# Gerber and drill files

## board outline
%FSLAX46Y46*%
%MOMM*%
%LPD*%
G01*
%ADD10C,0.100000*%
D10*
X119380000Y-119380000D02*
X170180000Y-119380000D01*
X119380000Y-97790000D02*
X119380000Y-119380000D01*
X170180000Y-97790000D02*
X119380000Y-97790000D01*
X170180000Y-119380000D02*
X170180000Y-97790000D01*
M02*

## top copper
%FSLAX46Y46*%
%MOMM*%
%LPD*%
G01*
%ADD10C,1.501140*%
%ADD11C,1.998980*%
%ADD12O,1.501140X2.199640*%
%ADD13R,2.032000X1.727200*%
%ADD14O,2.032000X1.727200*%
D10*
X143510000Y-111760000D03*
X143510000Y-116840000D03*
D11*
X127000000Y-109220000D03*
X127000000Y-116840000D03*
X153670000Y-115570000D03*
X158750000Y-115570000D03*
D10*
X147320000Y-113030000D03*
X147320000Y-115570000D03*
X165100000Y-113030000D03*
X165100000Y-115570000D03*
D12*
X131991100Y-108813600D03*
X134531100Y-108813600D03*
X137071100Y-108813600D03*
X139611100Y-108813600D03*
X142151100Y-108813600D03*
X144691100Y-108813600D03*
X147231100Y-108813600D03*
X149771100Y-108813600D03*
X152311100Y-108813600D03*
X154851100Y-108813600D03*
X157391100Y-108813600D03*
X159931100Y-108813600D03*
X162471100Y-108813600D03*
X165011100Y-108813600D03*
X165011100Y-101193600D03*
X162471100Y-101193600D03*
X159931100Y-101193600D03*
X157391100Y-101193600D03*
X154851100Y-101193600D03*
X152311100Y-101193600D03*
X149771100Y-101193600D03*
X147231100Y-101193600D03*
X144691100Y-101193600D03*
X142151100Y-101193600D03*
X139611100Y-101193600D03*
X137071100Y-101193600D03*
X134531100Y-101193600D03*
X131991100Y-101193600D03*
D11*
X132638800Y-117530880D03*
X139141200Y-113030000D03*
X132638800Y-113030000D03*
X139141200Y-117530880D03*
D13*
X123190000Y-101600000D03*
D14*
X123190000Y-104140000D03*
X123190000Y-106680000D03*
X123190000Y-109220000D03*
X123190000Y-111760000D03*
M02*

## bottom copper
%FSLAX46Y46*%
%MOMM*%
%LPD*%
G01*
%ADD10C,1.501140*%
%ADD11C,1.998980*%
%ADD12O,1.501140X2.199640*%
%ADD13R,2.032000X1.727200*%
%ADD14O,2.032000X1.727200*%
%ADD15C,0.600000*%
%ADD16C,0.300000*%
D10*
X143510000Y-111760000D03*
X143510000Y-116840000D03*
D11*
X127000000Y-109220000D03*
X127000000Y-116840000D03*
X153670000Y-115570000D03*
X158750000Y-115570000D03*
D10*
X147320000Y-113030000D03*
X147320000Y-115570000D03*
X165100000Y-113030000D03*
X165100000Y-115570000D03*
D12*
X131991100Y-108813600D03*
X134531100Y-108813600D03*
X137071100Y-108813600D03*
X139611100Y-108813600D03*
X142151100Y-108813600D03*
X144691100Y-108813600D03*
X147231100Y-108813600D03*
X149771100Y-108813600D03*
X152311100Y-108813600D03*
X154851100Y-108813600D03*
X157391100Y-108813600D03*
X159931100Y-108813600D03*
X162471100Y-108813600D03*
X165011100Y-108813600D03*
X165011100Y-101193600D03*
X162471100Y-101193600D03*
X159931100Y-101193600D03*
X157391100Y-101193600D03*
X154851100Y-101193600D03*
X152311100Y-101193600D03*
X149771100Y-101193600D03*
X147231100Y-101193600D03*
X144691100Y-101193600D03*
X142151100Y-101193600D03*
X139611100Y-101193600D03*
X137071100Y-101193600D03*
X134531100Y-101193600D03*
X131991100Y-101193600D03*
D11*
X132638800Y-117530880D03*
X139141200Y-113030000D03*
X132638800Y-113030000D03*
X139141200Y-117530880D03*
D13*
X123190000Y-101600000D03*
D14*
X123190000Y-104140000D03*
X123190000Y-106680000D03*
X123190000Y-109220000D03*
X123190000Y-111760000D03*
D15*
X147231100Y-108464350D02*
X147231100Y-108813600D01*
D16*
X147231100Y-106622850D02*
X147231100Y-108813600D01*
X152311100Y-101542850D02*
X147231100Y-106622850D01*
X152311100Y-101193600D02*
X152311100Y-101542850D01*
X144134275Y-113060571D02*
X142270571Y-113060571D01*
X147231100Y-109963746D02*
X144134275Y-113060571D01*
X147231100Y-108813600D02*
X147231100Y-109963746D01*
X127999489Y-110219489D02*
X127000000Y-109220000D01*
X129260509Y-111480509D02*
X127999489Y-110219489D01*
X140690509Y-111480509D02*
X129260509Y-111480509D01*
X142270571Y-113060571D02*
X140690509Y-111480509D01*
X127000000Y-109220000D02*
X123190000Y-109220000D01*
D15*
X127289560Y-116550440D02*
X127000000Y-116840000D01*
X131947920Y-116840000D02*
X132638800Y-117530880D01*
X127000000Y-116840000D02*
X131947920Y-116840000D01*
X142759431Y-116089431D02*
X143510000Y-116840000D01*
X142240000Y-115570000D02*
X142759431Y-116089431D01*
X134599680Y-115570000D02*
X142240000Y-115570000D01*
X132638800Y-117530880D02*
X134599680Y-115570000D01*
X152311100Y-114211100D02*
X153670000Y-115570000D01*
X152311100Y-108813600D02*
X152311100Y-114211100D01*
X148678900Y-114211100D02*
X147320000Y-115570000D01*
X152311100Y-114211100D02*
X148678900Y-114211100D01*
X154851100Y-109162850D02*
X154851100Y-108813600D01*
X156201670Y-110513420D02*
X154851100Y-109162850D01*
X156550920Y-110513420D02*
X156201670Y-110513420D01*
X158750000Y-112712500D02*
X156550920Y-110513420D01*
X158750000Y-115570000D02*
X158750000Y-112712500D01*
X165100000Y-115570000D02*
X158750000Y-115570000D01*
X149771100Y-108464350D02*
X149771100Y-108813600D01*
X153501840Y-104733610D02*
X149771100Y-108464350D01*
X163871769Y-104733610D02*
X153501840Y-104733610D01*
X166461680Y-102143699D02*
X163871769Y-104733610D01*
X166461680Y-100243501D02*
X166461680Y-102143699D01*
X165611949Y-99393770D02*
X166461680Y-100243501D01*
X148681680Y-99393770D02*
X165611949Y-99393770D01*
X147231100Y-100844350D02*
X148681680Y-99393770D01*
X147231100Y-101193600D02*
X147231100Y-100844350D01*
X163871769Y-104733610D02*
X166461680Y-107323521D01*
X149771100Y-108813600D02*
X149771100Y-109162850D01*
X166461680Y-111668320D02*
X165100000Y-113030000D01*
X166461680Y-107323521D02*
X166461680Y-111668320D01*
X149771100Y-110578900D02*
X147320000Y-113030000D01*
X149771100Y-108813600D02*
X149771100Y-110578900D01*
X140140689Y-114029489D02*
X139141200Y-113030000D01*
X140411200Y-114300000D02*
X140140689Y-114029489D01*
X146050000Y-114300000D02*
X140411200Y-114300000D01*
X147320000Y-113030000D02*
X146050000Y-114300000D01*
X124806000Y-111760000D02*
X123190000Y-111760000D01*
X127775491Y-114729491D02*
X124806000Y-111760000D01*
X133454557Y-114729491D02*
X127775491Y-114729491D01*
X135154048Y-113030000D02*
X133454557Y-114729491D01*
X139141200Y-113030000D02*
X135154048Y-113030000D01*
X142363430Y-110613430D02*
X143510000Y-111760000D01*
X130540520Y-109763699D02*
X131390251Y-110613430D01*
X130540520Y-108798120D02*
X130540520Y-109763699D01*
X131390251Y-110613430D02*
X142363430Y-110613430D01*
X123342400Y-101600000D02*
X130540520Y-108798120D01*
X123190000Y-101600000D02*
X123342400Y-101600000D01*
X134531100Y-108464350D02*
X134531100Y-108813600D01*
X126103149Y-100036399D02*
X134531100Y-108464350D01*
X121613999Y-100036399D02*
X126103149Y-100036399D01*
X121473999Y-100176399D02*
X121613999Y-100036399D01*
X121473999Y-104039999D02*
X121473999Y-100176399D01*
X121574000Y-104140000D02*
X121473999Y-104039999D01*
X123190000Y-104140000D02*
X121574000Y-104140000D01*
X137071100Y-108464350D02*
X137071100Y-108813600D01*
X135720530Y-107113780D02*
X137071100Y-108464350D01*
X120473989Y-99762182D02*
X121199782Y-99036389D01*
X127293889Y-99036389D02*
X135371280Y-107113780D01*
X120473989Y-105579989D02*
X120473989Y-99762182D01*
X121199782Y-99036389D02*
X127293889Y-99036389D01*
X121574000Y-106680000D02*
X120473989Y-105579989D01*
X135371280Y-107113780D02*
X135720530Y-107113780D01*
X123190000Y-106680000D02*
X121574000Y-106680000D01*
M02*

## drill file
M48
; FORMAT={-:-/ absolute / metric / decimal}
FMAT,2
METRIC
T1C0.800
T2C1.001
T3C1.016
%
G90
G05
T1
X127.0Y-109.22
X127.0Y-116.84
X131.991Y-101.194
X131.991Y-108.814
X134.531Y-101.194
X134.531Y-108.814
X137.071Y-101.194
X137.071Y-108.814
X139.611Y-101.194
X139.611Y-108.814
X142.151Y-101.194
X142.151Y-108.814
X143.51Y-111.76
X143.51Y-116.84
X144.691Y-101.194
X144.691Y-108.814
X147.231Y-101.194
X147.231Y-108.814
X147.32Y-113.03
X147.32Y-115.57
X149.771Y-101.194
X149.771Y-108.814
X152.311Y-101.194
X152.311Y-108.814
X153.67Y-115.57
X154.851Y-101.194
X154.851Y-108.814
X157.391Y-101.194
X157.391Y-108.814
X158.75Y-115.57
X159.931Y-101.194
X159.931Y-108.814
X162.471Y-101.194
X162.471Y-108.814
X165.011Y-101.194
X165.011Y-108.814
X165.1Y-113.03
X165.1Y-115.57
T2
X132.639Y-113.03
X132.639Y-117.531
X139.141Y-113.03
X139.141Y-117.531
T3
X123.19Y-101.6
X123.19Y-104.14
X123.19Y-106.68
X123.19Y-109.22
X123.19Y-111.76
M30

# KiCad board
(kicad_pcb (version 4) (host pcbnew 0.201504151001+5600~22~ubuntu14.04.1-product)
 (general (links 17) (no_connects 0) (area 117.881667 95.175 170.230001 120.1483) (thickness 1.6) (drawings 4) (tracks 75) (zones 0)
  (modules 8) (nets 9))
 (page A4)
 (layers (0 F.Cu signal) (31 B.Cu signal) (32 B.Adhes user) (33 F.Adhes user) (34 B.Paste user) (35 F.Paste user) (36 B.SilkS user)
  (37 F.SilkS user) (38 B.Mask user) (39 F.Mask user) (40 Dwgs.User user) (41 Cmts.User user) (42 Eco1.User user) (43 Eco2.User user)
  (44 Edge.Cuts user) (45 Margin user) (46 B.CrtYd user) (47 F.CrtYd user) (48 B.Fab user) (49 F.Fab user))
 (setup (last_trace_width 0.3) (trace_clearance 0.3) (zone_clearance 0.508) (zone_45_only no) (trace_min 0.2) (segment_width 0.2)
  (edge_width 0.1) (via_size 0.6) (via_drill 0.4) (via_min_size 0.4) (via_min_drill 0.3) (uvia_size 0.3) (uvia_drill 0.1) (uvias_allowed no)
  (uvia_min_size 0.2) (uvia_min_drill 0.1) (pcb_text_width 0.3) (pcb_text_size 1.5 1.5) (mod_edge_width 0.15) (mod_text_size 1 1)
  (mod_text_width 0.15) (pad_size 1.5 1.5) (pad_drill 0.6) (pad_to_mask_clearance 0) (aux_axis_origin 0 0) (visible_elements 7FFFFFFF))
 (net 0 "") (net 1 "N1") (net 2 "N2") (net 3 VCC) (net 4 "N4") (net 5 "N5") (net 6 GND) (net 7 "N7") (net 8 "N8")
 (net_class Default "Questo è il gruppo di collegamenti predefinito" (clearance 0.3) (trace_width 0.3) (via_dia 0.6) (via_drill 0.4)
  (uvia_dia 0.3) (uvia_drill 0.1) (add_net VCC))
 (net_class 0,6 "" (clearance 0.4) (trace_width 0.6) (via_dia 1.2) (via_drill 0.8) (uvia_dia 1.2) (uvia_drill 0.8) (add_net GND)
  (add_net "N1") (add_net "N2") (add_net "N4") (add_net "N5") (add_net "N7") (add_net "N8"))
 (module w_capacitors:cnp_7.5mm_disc (layer F.Cu) (at 143.51 114.3 270)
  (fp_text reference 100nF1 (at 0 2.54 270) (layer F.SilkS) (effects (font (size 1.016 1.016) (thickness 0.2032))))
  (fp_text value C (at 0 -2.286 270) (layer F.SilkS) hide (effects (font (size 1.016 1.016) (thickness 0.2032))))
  (pad 1 thru_hole circle (at -2.54 0 270) (size 1.50114 1.50114) (drill 0.8001) (layers *.Cu *.Mask F.SilkS) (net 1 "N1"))
  (pad 2 thru_hole circle (at 2.54 0 270) (size 1.50114 1.50114) (drill 0.8001) (layers *.Cu *.Mask F.SilkS) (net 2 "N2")))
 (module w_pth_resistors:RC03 (layer F.Cu) (at 127 113.03 270) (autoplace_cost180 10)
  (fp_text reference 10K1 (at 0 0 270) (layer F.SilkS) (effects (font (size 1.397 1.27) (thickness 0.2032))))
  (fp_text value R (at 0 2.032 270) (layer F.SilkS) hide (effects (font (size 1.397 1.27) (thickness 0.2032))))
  (pad 1 thru_hole circle (at -3.81 0 270) (size 1.99898 1.99898) (drill 0.8001) (layers *.Cu *.Mask F.SilkS) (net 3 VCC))
  (pad 2 thru_hole circle (at 3.81 0 270) (size 1.99898 1.99898) (drill 0.8001) (layers *.Cu *.Mask F.SilkS) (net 2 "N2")))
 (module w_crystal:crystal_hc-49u (layer F.Cu) (at 156.21 115.57) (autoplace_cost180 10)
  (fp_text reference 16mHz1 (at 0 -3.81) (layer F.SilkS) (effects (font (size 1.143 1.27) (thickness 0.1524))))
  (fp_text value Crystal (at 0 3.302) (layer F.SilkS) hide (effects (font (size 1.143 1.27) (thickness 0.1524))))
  (pad 1 thru_hole circle (at -2.54 0) (size 1.99898 1.99898) (drill 0.8001) (layers *.Cu *.Mask F.SilkS) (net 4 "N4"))
  (pad 2 thru_hole circle (at 2.54 0) (size 1.99898 1.99898) (drill 0.8001) (layers *.Cu *.Mask F.SilkS) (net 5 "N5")))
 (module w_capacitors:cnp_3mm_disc (layer F.Cu) (at 147.32 114.3 270)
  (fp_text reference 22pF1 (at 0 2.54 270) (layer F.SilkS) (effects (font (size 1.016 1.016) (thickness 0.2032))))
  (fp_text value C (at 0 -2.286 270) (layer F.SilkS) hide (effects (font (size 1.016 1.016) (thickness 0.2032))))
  (pad 1 thru_hole circle (at -1.27 0 270) (size 1.50114 1.50114) (drill 0.8001) (layers *.Cu *.Mask F.SilkS) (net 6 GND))
  (pad 2 thru_hole circle (at 1.27 0 270) (size 1.50114 1.50114) (drill 0.8001) (layers *.Cu *.Mask F.SilkS) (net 4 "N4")))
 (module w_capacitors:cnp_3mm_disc (layer F.Cu) (at 165.1 114.3 270)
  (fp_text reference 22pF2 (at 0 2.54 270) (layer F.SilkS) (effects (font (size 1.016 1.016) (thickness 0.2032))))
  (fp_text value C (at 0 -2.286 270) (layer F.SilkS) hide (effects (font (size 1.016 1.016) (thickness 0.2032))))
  (pad 1 thru_hole circle (at -1.27 0 270) (size 1.50114 1.50114) (drill 0.8001) (layers *.Cu *.Mask F.SilkS) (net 6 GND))
  (pad 2 thru_hole circle (at 1.27 0 270) (size 1.50114 1.50114) (drill 0.8001) (layers *.Cu *.Mask F.SilkS) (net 5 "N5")))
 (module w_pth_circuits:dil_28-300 (layer F.Cu) (at 148.5011 105.0036)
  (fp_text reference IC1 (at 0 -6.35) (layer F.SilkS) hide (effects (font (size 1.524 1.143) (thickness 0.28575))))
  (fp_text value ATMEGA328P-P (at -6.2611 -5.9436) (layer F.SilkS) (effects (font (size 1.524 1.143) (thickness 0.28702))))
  (pad 1 thru_hole oval (at -16.51 3.81) (size 1.50114 2.19964) (drill 0.8001) (layers *.Cu *.Mask F.SilkS))
  (pad 2 thru_hole oval (at -13.97 3.81) (size 1.50114 2.19964) (drill 0.8001) (layers *.Cu *.Mask F.SilkS) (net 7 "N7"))
  (pad 3 thru_hole oval (at -11.43 3.81) (size 1.50114 2.19964) (drill 0.8001) (layers *.Cu *.Mask F.SilkS) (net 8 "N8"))
  (pad 4 thru_hole oval (at -8.89 3.81) (size 1.50114 2.19964) (drill 0.8001) (layers *.Cu *.Mask F.SilkS))
  (pad 5 thru_hole oval (at -6.35 3.81) (size 1.50114 2.19964) (drill 0.8001) (layers *.Cu *.Mask F.SilkS))
  (pad 6 thru_hole oval (at -3.81 3.81) (size 1.50114 2.19964) (drill 0.8001) (layers *.Cu *.Mask F.SilkS))
  (pad 7 thru_hole oval (at -1.27 3.81) (size 1.50114 2.19964) (drill 0.8001) (layers *.Cu *.Mask F.SilkS) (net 3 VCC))
  (pad 8 thru_hole oval (at 1.27 3.81) (size 1.50114 2.19964) (drill 0.8001) (layers *.Cu *.Mask F.SilkS) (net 6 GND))
  (pad 9 thru_hole oval (at 3.81 3.81) (size 1.50114 2.19964) (drill 0.8001) (layers *.Cu *.Mask F.SilkS) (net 4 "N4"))
  (pad 10 thru_hole oval (at 6.35 3.81) (size 1.50114 2.19964) (drill 0.8001) (layers *.Cu *.Mask F.SilkS) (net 5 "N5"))
  (pad 11 thru_hole oval (at 8.89 3.81) (size 1.50114 2.19964) (drill 0.8001) (layers *.Cu *.Mask F.SilkS))
  (pad 12 thru_hole oval (at 11.43 3.81) (size 1.50114 2.19964) (drill 0.8001) (layers *.Cu *.Mask F.SilkS))
  (pad 13 thru_hole oval (at 13.97 3.81) (size 1.50114 2.19964) (drill 0.8001) (layers *.Cu *.Mask F.SilkS))
  (pad 14 thru_hole oval (at 16.51 3.81) (size 1.50114 2.19964) (drill 0.8001) (layers *.Cu *.Mask F.SilkS))
  (pad 15 thru_hole oval (at 16.51 -3.81) (size 1.50114 2.19964) (drill 0.8001) (layers *.Cu *.Mask F.SilkS))
  (pad 16 thru_hole oval (at 13.97 -3.81) (size 1.50114 2.19964) (drill 0.8001) (layers *.Cu *.Mask F.SilkS))
  (pad 17 thru_hole oval (at 11.43 -3.81) (size 1.50114 2.19964) (drill 0.8001) (layers *.Cu *.Mask F.SilkS))
  (pad 18 thru_hole oval (at 8.89 -3.81) (size 1.50114 2.19964) (drill 0.8001) (layers *.Cu *.Mask F.SilkS))
  (pad 19 thru_hole oval (at 6.35 -3.81) (size 1.50114 2.19964) (drill 0.8001) (layers *.Cu *.Mask F.SilkS))
  (pad 20 thru_hole oval (at 3.81 -3.81) (size 1.50114 2.19964) (drill 0.8001) (layers *.Cu *.Mask F.SilkS) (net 3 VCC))
  (pad 21 thru_hole oval (at 1.27 -3.81) (size 1.50114 2.19964) (drill 0.8001) (layers *.Cu *.Mask F.SilkS))
  (pad 22 thru_hole oval (at -1.27 -3.81) (size 1.50114 2.19964) (drill 0.8001) (layers *.Cu *.Mask F.SilkS) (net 6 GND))
  (pad 23 thru_hole oval (at -3.81 -3.81) (size 1.50114 2.19964) (drill 0.8001) (layers *.Cu *.Mask F.SilkS))
  (pad 24 thru_hole oval (at -6.35 -3.81) (size 1.50114 2.19964) (drill 0.8001) (layers *.Cu *.Mask F.SilkS))
  (pad 25 thru_hole oval (at -8.89 -3.81) (size 1.50114 2.19964) (drill 0.8001) (layers *.Cu *.Mask F.SilkS))
  (pad 26 thru_hole oval (at -11.43 -3.81) (size 1.50114 2.19964) (drill 0.8001) (layers *.Cu *.Mask F.SilkS))
  (pad 27 thru_hole oval (at -13.97 -3.81) (size 1.50114 2.19964) (drill 0.8001) (layers *.Cu *.Mask F.SilkS))
  (pad 28 thru_hole oval (at -16.51 -3.81) (size 1.50114 2.19964) (drill 0.8001) (layers *.Cu *.Mask F.SilkS)))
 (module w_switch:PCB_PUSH (layer F.Cu) (at 135.89 115.28044 90)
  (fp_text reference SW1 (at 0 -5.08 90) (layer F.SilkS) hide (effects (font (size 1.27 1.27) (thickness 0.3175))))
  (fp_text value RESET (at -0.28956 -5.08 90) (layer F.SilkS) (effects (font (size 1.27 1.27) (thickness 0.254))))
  (pad 1 thru_hole circle (at -2.25044 -3.2512 90) (size 1.99898 1.99898) (drill 1.00076) (layers *.Cu *.Mask F.SilkS) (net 2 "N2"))
  (pad 2 thru_hole circle (at 2.25044 3.2512 90) (size 1.99898 1.99898) (drill 1.00076) (layers *.Cu *.Mask F.SilkS) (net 6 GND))
  (pad 4 thru_hole circle (at 2.25044 -3.2512 90) (size 1.99898 1.99898) (drill 1.00076) (layers *.Cu *.Mask F.SilkS))
  (pad 3 thru_hole circle (at -2.25044 3.2512 90) (size 1.99898 1.99898) (drill 1.00076) (layers *.Cu *.Mask F.SilkS)))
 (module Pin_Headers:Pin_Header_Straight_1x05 (layer F.Cu) (at 123.19 101.6)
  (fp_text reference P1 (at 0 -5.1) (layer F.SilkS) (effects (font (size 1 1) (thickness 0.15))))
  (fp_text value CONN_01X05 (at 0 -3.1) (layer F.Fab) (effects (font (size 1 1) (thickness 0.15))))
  (pad 1 thru_hole rect (at 0 0) (size 2.032 1.7272) (drill 1.016) (layers *.Cu *.Mask F.SilkS) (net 1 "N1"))
  (pad 2 thru_hole oval (at 0 2.54) (size 2.032 1.7272) (drill 1.016) (layers *.Cu *.Mask F.SilkS) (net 7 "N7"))
  (pad 3 thru_hole oval (at 0 5.08) (size 2.032 1.7272) (drill 1.016) (layers *.Cu *.Mask F.SilkS) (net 8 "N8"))
  (pad 4 thru_hole oval (at 0 7.62) (size 2.032 1.7272) (drill 1.016) (layers *.Cu *.Mask F.SilkS) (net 3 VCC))
  (pad 5 thru_hole oval (at 0 10.16) (size 2.032 1.7272) (drill 1.016) (layers *.Cu *.Mask F.SilkS) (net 6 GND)))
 (gr_line (start 119.38 119.38) (end 170.18 119.38) (layer Edge.Cuts) (width 0.1))
 (gr_line (start 119.38 97.79) (end 119.38 119.38) (layer Edge.Cuts) (width 0.1))
 (gr_line (start 170.18 97.79) (end 119.38 97.79) (layer Edge.Cuts) (width 0.1))
 (gr_line (start 170.18 119.38) (end 170.18 97.79) (layer Edge.Cuts) (width 0.1))
 (segment (start 147.2311 108.46435) (end 147.2311 108.8136) (width 0.6) (layer B.Cu) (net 3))
 (segment (start 147.2311 106.62285) (end 147.2311 108.8136) (width 0.3) (layer B.Cu) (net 3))
 (segment (start 152.3111 101.54285) (end 147.2311 106.62285) (width 0.3) (layer B.Cu) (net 3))
 (segment (start 152.3111 101.1936) (end 152.3111 101.54285) (width 0.3) (layer B.Cu) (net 3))
 (segment (start 144.134275 113.060571) (end 142.270571 113.060571) (width 0.3) (layer B.Cu) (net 3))
 (segment (start 147.2311 109.963746) (end 144.134275 113.060571) (width 0.3) (layer B.Cu) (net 3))
 (segment (start 147.2311 108.8136) (end 147.2311 109.963746) (width 0.3) (layer B.Cu) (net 3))
 (segment (start 127.999489 110.219489) (end 127 109.22) (width 0.3) (layer B.Cu) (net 3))
 (segment (start 129.260509 111.480509) (end 127.999489 110.219489) (width 0.3) (layer B.Cu) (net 3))
 (segment (start 140.690509 111.480509) (end 129.260509 111.480509) (width 0.3) (layer B.Cu) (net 3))
 (segment (start 142.270571 113.060571) (end 140.690509 111.480509) (width 0.3) (layer B.Cu) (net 3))
 (segment (start 127 109.22) (end 123.19 109.22) (width 0.3) (layer B.Cu) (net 3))
 (segment (start 127.28956 116.55044) (end 127 116.84) (width 0.6) (layer B.Cu) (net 2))
 (segment (start 131.94792 116.84) (end 132.6388 117.53088) (width 0.6) (layer B.Cu) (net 2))
 (segment (start 127 116.84) (end 131.94792 116.84) (width 0.6) (layer B.Cu) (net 2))
 (segment (start 142.759431 116.089431) (end 143.51 116.84) (width 0.6) (layer B.Cu) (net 2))
 (segment (start 142.24 115.57) (end 142.759431 116.089431) (width 0.6) (layer B.Cu) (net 2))
 (segment (start 134.59968 115.57) (end 142.24 115.57) (width 0.6) (layer B.Cu) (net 2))
 (segment (start 132.6388 117.53088) (end 134.59968 115.57) (width 0.6) (layer B.Cu) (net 2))
 (segment (start 152.3111 114.2111) (end 153.67 115.57) (width 0.6) (layer B.Cu) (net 4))
 (segment (start 152.3111 108.8136) (end 152.3111 114.2111) (width 0.6) (layer B.Cu) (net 4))
 (segment (start 148.6789 114.2111) (end 147.32 115.57) (width 0.6) (layer B.Cu) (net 4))
 (segment (start 152.3111 114.2111) (end 148.6789 114.2111) (width 0.6) (layer B.Cu) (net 4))
 (segment (start 154.8511 109.16285) (end 154.8511 108.8136) (width 0.6) (layer B.Cu) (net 5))
 (segment (start 156.20167 110.51342) (end 154.8511 109.16285) (width 0.6) (layer B.Cu) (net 5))
 (segment (start 156.55092 110.51342) (end 156.20167 110.51342) (width 0.6) (layer B.Cu) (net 5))
 (segment (start 158.75 112.7125) (end 156.55092 110.51342) (width 0.6) (layer B.Cu) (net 5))
 (segment (start 158.75 115.57) (end 158.75 112.7125) (width 0.6) (layer B.Cu) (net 5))
 (segment (start 165.1 115.57) (end 158.75 115.57) (width 0.6) (layer B.Cu) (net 5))
 (segment (start 149.7711 108.46435) (end 149.7711 108.8136) (width 0.6) (layer B.Cu) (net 6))
 (segment (start 153.50184 104.73361) (end 149.7711 108.46435) (width 0.6) (layer B.Cu) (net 6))
 (segment (start 163.871769 104.73361) (end 153.50184 104.73361) (width 0.6) (layer B.Cu) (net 6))
 (segment (start 166.46168 102.143699) (end 163.871769 104.73361) (width 0.6) (layer B.Cu) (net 6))
 (segment (start 166.46168 100.243501) (end 166.46168 102.143699) (width 0.6) (layer B.Cu) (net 6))
 (segment (start 165.611949 99.39377) (end 166.46168 100.243501) (width 0.6) (layer B.Cu) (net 6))
 (segment (start 148.68168 99.39377) (end 165.611949 99.39377) (width 0.6) (layer B.Cu) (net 6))
 (segment (start 147.2311 100.84435) (end 148.68168 99.39377) (width 0.6) (layer B.Cu) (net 6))
 (segment (start 147.2311 101.1936) (end 147.2311 100.84435) (width 0.6) (layer B.Cu) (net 6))
 (segment (start 163.871769 104.73361) (end 166.46168 107.323521) (width 0.6) (layer B.Cu) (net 6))
 (segment (start 149.7711 108.8136) (end 149.7711 109.16285) (width 0.6) (layer B.Cu) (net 6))
 (segment (start 166.46168 111.66832) (end 165.1 113.03) (width 0.6) (layer B.Cu) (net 6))
 (segment (start 166.46168 107.323521) (end 166.46168 111.66832) (width 0.6) (layer B.Cu) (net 6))
 (segment (start 149.7711 110.5789) (end 147.32 113.03) (width 0.6) (layer B.Cu) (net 6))
 (segment (start 149.7711 108.8136) (end 149.7711 110.5789) (width 0.6) (layer B.Cu) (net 6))
 (segment (start 140.140689 114.029489) (end 139.1412 113.03) (width 0.6) (layer B.Cu) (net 6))
 (segment (start 140.4112 114.3) (end 140.140689 114.029489) (width 0.6) (layer B.Cu) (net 6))
 (segment (start 146.05 114.3) (end 140.4112 114.3) (width 0.6) (layer B.Cu) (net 6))
 (segment (start 147.32 113.03) (end 146.05 114.3) (width 0.6) (layer B.Cu) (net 6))
 (segment (start 124.806 111.76) (end 123.19 111.76) (width 0.6) (layer B.Cu) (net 6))
 (segment (start 127.775491 114.729491) (end 124.806 111.76) (width 0.6) (layer B.Cu) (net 6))
 (segment (start 133.454557 114.729491) (end 127.775491 114.729491) (width 0.6) (layer B.Cu) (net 6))
 (segment (start 135.154048 113.03) (end 133.454557 114.729491) (width 0.6) (layer B.Cu) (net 6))
 (segment (start 139.1412 113.03) (end 135.154048 113.03) (width 0.6) (layer B.Cu) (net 6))
 (segment (start 142.36343 110.61343) (end 143.51 111.76) (width 0.6) (layer B.Cu) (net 1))
 (segment (start 130.54052 109.763699) (end 131.390251 110.61343) (width 0.6) (layer B.Cu) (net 1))
 (segment (start 130.54052 108.79812) (end 130.54052 109.763699) (width 0.6) (layer B.Cu) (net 1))
 (segment (start 131.390251 110.61343) (end 142.36343 110.61343) (width 0.6) (layer B.Cu) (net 1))
 (segment (start 123.3424 101.6) (end 130.54052 108.79812) (width 0.6) (layer B.Cu) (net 1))
 (segment (start 123.19 101.6) (end 123.3424 101.6) (width 0.6) (layer B.Cu) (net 1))
 (segment (start 134.5311 108.46435) (end 134.5311 108.8136) (width 0.6) (layer B.Cu) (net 7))
 (segment (start 126.103149 100.036399) (end 134.5311 108.46435) (width 0.6) (layer B.Cu) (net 7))
 (segment (start 121.613999 100.036399) (end 126.103149 100.036399) (width 0.6) (layer B.Cu) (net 7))
 (segment (start 121.473999 100.176399) (end 121.613999 100.036399) (width 0.6) (layer B.Cu) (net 7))
 (segment (start 121.473999 104.039999) (end 121.473999 100.176399) (width 0.6) (layer B.Cu) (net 7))
 (segment (start 121.574 104.14) (end 121.473999 104.039999) (width 0.6) (layer B.Cu) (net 7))
 (segment (start 123.19 104.14) (end 121.574 104.14) (width 0.6) (layer B.Cu) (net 7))
 (segment (start 137.0711 108.46435) (end 137.0711 108.8136) (width 0.6) (layer B.Cu) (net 8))
 (segment (start 135.72053 107.11378) (end 137.0711 108.46435) (width 0.6) (layer B.Cu) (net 8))
 (segment (start 120.473989 99.762182) (end 121.199782 99.036389) (width 0.6) (layer B.Cu) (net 8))
 (segment (start 127.293889 99.036389) (end 135.37128 107.11378) (width 0.6) (layer B.Cu) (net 8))
 (segment (start 120.473989 105.579989) (end 120.473989 99.762182) (width 0.6) (layer B.Cu) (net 8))
 (segment (start 121.199782 99.036389) (end 127.293889 99.036389) (width 0.6) (layer B.Cu) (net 8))
 (segment (start 121.574 106.68) (end 120.473989 105.579989) (width 0.6) (layer B.Cu) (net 8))
 (segment (start 135.37128 107.11378) (end 135.72053 107.11378) (width 0.6) (layer B.Cu) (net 8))
 (segment (start 123.19 106.68) (end 121.574 106.68) (width 0.6) (layer B.Cu) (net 8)))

